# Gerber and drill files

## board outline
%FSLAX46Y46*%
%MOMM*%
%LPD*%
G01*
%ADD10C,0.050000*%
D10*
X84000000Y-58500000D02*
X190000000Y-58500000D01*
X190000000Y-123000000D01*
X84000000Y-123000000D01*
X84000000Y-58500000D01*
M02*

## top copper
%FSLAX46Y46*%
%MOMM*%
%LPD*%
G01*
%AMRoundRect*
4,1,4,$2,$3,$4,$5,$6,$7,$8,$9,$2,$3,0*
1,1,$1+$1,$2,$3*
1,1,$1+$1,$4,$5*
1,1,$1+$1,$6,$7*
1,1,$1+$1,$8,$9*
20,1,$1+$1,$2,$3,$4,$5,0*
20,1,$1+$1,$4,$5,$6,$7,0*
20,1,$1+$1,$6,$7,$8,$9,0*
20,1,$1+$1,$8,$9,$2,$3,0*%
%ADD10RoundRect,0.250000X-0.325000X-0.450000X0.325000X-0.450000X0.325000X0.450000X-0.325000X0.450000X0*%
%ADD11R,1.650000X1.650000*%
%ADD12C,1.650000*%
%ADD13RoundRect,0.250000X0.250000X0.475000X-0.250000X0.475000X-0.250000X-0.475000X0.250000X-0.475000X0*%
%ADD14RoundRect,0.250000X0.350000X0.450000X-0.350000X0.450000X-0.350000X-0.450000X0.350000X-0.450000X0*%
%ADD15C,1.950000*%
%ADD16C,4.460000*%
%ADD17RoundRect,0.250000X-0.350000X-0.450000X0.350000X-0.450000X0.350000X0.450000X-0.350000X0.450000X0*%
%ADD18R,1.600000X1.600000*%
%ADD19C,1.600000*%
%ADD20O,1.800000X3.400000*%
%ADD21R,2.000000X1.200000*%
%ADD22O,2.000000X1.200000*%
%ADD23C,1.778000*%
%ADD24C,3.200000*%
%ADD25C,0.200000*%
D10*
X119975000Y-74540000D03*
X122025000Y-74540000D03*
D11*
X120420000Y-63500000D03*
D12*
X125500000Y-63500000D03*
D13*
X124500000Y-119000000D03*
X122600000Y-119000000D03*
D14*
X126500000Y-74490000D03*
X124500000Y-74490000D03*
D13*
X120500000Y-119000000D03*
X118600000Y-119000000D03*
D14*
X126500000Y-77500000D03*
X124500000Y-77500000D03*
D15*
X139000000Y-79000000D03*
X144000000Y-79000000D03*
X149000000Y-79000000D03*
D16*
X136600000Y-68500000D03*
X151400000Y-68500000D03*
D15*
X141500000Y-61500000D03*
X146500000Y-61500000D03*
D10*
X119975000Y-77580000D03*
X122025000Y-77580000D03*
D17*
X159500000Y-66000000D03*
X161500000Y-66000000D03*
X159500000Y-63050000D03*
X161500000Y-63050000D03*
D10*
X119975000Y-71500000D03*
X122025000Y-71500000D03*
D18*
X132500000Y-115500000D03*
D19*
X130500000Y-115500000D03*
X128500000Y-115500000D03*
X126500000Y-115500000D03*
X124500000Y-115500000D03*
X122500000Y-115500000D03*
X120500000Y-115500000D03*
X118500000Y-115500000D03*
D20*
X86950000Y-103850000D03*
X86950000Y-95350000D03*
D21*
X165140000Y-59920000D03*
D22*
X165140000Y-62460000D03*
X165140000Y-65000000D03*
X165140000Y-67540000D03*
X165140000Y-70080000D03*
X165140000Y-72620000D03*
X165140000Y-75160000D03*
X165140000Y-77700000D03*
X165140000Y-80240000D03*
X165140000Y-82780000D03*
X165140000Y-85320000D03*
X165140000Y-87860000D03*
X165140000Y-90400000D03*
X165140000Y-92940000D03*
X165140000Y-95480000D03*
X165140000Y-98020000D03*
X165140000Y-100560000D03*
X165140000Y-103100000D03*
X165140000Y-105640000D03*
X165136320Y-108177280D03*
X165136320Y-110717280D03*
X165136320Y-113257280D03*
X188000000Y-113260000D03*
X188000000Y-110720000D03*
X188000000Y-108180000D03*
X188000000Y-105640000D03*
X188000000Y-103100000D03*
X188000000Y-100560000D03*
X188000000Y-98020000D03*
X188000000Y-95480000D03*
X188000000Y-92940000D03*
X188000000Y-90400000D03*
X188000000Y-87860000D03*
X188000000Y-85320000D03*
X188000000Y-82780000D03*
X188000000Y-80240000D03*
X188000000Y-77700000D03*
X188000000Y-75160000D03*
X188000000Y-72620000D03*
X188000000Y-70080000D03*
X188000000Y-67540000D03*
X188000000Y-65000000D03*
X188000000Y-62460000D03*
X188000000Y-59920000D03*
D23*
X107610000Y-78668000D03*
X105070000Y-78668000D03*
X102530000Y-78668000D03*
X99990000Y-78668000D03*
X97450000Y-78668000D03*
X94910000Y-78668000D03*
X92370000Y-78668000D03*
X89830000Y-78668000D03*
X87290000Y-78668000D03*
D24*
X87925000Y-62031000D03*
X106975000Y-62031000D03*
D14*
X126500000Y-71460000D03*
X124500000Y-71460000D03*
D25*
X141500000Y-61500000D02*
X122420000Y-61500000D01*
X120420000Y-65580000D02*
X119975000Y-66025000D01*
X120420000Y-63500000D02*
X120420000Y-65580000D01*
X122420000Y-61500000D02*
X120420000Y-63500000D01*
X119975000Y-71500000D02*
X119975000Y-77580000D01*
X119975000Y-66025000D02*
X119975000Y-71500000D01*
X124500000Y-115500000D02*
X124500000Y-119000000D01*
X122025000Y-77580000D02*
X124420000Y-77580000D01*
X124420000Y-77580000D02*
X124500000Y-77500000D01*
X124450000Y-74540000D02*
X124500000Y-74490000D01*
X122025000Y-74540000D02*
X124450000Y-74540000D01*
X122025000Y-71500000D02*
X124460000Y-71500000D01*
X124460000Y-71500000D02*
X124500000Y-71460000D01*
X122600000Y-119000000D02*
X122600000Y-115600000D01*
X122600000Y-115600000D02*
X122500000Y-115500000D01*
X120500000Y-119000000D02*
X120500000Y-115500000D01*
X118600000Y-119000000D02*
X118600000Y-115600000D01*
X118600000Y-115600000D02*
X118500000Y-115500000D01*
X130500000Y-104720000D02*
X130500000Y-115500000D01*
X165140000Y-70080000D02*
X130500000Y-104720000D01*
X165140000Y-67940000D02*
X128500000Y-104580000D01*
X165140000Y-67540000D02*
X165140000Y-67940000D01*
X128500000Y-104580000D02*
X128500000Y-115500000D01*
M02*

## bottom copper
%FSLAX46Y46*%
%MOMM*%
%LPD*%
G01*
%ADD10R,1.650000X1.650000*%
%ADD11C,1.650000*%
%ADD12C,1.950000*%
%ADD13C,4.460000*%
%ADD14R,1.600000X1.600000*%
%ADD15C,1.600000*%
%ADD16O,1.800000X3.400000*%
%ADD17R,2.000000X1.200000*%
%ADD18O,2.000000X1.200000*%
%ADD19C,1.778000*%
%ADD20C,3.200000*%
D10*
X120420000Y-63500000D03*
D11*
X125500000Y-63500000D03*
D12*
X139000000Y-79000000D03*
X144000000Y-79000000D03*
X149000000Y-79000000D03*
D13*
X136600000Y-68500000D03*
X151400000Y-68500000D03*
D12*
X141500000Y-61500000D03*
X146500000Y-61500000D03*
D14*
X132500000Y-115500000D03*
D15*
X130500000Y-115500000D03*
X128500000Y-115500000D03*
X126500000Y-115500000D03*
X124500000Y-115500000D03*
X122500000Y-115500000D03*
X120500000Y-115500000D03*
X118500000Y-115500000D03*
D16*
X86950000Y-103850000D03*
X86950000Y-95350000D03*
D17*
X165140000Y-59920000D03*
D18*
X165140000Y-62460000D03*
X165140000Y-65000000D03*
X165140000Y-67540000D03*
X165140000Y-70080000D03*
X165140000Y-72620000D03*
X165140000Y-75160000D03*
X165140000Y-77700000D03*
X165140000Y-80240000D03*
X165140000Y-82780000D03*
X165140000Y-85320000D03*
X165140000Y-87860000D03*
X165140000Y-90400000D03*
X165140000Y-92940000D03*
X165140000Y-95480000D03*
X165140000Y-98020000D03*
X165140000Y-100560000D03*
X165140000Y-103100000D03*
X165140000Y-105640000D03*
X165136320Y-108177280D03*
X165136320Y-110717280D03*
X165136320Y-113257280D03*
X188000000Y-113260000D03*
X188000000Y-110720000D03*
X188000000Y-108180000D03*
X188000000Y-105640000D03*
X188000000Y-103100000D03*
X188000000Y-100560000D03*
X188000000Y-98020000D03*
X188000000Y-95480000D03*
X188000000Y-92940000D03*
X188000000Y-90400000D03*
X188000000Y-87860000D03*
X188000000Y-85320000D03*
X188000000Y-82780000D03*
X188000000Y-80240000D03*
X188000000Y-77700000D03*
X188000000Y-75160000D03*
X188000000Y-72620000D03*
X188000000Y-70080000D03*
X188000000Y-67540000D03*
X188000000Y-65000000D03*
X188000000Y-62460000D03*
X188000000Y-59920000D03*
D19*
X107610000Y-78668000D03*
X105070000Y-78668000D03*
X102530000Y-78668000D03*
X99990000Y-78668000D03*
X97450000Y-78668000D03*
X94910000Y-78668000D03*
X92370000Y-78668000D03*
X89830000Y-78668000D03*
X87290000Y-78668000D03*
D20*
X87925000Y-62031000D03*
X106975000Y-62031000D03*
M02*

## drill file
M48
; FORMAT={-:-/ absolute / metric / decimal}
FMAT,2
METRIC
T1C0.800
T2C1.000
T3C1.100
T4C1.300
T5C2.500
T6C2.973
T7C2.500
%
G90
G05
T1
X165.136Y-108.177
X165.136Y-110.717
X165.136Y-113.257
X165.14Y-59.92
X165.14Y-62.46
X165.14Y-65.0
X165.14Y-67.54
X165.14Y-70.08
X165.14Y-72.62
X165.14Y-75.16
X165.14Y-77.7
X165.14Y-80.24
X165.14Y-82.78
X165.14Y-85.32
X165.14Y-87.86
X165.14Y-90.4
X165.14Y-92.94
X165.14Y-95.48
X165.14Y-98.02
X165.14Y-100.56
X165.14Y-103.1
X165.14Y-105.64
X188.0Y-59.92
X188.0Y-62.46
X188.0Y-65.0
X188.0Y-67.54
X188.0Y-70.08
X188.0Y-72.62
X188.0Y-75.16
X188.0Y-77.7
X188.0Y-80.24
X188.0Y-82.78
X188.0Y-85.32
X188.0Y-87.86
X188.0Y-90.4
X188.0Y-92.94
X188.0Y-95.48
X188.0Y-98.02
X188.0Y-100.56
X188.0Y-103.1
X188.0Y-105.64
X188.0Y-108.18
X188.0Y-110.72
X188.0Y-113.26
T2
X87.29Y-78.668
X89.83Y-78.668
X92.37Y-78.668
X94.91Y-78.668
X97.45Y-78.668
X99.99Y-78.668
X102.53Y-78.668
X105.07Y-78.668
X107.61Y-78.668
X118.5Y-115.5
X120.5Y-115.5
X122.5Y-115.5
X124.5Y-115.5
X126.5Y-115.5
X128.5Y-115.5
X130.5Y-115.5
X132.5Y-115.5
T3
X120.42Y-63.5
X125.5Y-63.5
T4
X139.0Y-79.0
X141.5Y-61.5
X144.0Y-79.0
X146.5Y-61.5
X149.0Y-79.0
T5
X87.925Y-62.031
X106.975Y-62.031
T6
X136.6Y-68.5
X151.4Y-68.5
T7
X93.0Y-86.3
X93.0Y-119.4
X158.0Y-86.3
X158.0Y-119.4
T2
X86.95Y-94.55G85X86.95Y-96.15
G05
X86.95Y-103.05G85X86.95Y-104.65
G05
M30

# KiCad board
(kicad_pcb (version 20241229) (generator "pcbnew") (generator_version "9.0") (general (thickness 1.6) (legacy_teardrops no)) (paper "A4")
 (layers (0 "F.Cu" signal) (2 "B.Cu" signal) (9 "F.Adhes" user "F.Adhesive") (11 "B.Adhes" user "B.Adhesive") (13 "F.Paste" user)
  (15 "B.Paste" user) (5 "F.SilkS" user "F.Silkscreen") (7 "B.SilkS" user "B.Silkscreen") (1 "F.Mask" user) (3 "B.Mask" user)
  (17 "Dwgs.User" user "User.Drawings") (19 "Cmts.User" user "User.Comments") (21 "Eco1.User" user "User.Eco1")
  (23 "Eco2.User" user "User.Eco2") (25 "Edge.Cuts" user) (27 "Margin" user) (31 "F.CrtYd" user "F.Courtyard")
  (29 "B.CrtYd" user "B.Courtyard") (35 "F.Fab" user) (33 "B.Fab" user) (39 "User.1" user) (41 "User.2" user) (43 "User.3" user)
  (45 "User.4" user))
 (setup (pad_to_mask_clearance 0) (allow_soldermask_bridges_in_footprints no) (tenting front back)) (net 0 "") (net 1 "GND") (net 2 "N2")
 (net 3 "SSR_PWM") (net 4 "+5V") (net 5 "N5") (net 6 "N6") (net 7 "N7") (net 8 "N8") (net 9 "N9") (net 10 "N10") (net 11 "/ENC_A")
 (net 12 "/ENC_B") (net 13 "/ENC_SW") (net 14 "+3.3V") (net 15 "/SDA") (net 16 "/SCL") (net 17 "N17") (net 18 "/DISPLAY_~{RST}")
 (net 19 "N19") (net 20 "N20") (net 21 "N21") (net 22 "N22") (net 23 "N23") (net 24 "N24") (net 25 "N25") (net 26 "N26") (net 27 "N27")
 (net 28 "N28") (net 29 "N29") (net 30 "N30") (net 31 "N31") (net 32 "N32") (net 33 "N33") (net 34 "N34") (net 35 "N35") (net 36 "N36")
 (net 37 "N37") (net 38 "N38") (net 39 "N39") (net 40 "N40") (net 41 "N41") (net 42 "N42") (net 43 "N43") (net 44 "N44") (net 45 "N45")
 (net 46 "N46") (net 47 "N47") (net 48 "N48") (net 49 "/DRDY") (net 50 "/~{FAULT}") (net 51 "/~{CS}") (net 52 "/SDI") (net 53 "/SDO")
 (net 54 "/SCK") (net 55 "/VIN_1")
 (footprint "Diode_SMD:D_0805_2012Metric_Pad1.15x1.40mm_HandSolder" (layer "F.Cu") (at 121 74.54)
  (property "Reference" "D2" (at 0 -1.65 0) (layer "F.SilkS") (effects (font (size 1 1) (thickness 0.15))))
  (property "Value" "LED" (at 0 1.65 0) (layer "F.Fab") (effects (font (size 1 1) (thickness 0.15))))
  (pad "1" smd roundrect (at -1.025 0) (size 1.15 1.4) (layers "F.Cu" "F.Mask" "F.Paste") (roundrect_rratio 0.217391) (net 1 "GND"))
  (pad "2" smd roundrect (at 1.025 0) (size 1.15 1.4) (layers "F.Cu" "F.Mask" "F.Paste") (roundrect_rratio 0.217391) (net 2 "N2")))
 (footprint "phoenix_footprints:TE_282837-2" (layer "F.Cu") (at 122.96 63.5)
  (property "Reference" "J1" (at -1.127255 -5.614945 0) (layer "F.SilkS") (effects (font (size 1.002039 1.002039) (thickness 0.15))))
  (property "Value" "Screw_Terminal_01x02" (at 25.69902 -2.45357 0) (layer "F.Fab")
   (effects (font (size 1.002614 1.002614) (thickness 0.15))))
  (pad "1" thru_hole rect (at -2.54 0) (size 1.65 1.65) (drill 1.1) (layers "*.Cu" "*.Mask") (remove_unused_layers no) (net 1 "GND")
   (solder_mask_margin 0.102))
  (pad "2" thru_hole circle (at 2.54 0) (size 1.65 1.65) (drill 1.1) (layers "*.Cu" "*.Mask") (remove_unused_layers no) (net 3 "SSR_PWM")
   (solder_mask_margin 0.102)))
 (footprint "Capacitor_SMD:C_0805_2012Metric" (layer "F.Cu") (at 123.55 119 180)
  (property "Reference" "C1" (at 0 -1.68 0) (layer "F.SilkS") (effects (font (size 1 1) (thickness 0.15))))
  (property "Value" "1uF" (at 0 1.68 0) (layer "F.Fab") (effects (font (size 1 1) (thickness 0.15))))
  (pad "1" smd roundrect (at -0.95 0 180) (size 1 1.45) (layers "F.Cu" "F.Mask" "F.Paste") (roundrect_rratio 0.25) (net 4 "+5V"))
  (pad "2" smd roundrect (at 0.95 0 180) (size 1 1.45) (layers "F.Cu" "F.Mask" "F.Paste") (roundrect_rratio 0.25) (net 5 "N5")))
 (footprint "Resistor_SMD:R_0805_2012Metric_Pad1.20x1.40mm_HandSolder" (layer "F.Cu") (at 125.5 74.49 180)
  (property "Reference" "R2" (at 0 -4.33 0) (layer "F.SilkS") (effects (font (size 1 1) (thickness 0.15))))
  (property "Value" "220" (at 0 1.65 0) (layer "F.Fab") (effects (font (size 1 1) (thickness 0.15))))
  (pad "1" smd roundrect (at -1 0 180) (size 1.2 1.4) (layers "F.Cu" "F.Mask" "F.Paste") (roundrect_rratio 0.208333) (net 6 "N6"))
  (pad "2" smd roundrect (at 1 0 180) (size 1.2 1.4) (layers "F.Cu" "F.Mask" "F.Paste") (roundrect_rratio 0.208333) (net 2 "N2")))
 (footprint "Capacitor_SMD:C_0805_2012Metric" (layer "F.Cu") (at 119.55 119 180)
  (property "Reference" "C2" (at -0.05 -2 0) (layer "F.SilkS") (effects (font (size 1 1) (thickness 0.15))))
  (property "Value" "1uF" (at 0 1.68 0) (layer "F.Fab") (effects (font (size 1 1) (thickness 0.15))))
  (pad "1" smd roundrect (at -0.95 0 180) (size 1 1.45) (layers "F.Cu" "F.Mask" "F.Paste") (roundrect_rratio 0.25) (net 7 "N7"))
  (pad "2" smd roundrect (at 0.95 0 180) (size 1 1.45) (layers "F.Cu" "F.Mask" "F.Paste") (roundrect_rratio 0.25) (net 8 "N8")))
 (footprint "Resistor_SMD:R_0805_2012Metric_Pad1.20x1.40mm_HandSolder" (layer "F.Cu") (at 125.5 77.5 180)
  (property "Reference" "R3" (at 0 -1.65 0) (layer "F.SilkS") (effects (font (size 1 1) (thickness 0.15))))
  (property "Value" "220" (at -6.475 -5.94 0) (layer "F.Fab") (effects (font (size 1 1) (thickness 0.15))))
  (pad "1" smd roundrect (at -1 0 180) (size 1.2 1.4) (layers "F.Cu" "F.Mask" "F.Paste") (roundrect_rratio 0.208333) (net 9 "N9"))
  (pad "2" smd roundrect (at 1 0 180) (size 1.2 1.4) (layers "F.Cu" "F.Mask" "F.Paste") (roundrect_rratio 0.208333) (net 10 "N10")))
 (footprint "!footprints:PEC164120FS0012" (layer "F.Cu") (at 139 79)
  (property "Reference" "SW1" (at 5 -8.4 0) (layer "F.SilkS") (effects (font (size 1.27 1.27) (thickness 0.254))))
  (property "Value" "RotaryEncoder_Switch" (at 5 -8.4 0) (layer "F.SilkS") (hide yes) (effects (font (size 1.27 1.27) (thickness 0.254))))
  (pad "A" thru_hole circle (at 0 0) (size 1.95 1.95) (drill 1.3) (layers "*.Cu" "*.Mask") (remove_unused_layers no) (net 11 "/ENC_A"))
  (pad "B" thru_hole circle (at 5 0) (size 1.95 1.95) (drill 1.3) (layers "*.Cu" "*.Mask") (remove_unused_layers no) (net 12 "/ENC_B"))
  (pad "C" thru_hole circle (at 10 0) (size 1.95 1.95) (drill 1.3) (layers "*.Cu" "*.Mask") (remove_unused_layers no) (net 1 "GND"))
  (pad "MH1" thru_hole circle (at -2.4 -10.5) (size 4.46 4.46) (drill 2.9732) (layers "*.Cu" "*.Mask") (remove_unused_layers no))
  (pad "MH2" thru_hole circle (at 12.4 -10.5) (size 4.46 4.46) (drill 2.9732) (layers "*.Cu" "*.Mask") (remove_unused_layers no))
  (pad "S1" thru_hole circle (at 2.5 -17.5) (size 1.95 1.95) (drill 1.3) (layers "*.Cu" "*.Mask") (remove_unused_layers no) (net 1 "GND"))
  (pad "S2" thru_hole circle (at 7.5 -17.5) (size 1.95 1.95) (drill 1.3) (layers "*.Cu" "*.Mask") (remove_unused_layers no)
   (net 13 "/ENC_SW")))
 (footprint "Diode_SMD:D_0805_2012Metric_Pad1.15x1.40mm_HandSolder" (layer "F.Cu") (at 121 77.58)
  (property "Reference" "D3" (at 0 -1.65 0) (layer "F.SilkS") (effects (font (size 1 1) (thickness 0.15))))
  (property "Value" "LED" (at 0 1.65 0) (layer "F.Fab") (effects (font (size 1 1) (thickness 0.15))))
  (pad "1" smd roundrect (at -1.025 0) (size 1.15 1.4) (layers "F.Cu" "F.Mask" "F.Paste") (roundrect_rratio 0.217391) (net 1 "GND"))
  (pad "2" smd roundrect (at 1.025 0) (size 1.15 1.4) (layers "F.Cu" "F.Mask" "F.Paste") (roundrect_rratio 0.217391) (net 10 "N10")))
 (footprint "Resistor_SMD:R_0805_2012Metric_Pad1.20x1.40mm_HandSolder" (layer "F.Cu") (at 160.5 66)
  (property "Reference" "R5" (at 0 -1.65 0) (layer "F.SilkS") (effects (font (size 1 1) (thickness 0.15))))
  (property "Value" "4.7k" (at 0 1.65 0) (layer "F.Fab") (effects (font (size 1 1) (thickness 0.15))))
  (pad "1" smd roundrect (at -1 0) (size 1.2 1.4) (layers "F.Cu" "F.Mask" "F.Paste") (roundrect_rratio 0.208333) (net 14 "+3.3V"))
  (pad "2" smd roundrect (at 1 0) (size 1.2 1.4) (layers "F.Cu" "F.Mask" "F.Paste") (roundrect_rratio 0.208333) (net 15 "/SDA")))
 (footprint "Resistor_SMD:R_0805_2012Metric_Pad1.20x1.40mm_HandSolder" (layer "F.Cu") (at 160.5 63.05)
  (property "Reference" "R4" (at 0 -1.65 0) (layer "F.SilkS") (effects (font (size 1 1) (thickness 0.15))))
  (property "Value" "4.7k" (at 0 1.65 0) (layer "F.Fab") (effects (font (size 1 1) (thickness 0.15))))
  (pad "1" smd roundrect (at -1 0) (size 1.2 1.4) (layers "F.Cu" "F.Mask" "F.Paste") (roundrect_rratio 0.208333) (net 14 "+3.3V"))
  (pad "2" smd roundrect (at 1 0) (size 1.2 1.4) (layers "F.Cu" "F.Mask" "F.Paste") (roundrect_rratio 0.208333) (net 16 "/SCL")))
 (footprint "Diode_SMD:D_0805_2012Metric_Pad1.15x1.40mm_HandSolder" (layer "F.Cu") (at 121 71.5)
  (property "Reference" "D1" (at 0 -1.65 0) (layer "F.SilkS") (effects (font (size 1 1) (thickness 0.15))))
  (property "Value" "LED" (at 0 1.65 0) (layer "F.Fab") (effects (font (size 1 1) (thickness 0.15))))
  (pad "1" smd roundrect (at -1.025 0) (size 1.15 1.4) (layers "F.Cu" "F.Mask" "F.Paste") (roundrect_rratio 0.217391) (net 1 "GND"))
  (pad "2" smd roundrect (at 1.025 0) (size 1.15 1.4) (layers "F.Cu" "F.Mask" "F.Paste") (roundrect_rratio 0.217391) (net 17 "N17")))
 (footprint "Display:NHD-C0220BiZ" (layer "F.Cu") (at 125.5 99.6)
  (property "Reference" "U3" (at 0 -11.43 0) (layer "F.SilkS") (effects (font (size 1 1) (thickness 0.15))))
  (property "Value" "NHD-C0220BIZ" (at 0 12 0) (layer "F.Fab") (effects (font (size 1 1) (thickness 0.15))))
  (pad "" np_thru_hole circle (at -32.5 -13.3) (size 2.5 2.5) (drill 2.5) (layers "*.Cu" "*.Mask"))
  (pad "" np_thru_hole circle (at -32.5 19.8) (size 2.5 2.5) (drill 2.5) (layers "*.Cu" "*.Mask"))
  (pad "" np_thru_hole circle (at 32.5 -13.3) (size 2.5 2.5) (drill 2.5) (layers "*.Cu" "*.Mask"))
  (pad "" np_thru_hole circle (at 32.5 19.8) (size 2.5 2.5) (drill 2.5) (layers "*.Cu" "*.Mask"))
  (pad "1" thru_hole rect (at 7 15.9) (size 1.6 1.6) (drill 1) (layers "*.Cu" "*.Mask") (remove_unused_layers no) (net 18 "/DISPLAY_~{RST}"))
  (pad "2" thru_hole circle (at 5 15.9) (size 1.6 1.6) (drill 1) (layers "*.Cu" "*.Mask") (remove_unused_layers no) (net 16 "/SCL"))
  (pad "3" thru_hole circle (at 3 15.9) (size 1.6 1.6) (drill 1) (layers "*.Cu" "*.Mask") (remove_unused_layers no) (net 15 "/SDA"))
  (pad "4" thru_hole circle (at 1 15.9) (size 1.6 1.6) (drill 1) (layers "*.Cu" "*.Mask") (remove_unused_layers no) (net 1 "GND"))
  (pad "5" thru_hole circle (at -1 15.9) (size 1.6 1.6) (drill 1) (layers "*.Cu" "*.Mask") (remove_unused_layers no) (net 4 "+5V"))
  (pad "6" thru_hole circle (at -3 15.9) (size 1.6 1.6) (drill 1) (layers "*.Cu" "*.Mask") (remove_unused_layers no) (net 5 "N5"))
  (pad "7" thru_hole circle (at -5 15.9) (size 1.6 1.6) (drill 1) (layers "*.Cu" "*.Mask") (remove_unused_layers no) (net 7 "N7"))
  (pad "8" thru_hole circle (at -7 15.9) (size 1.6 1.6) (drill 1) (layers "*.Cu" "*.Mask") (remove_unused_layers no) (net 8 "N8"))
  (pad "9" thru_hole oval (at -38.55 4.25) (size 1.8 3.4) (drill oval 1 2.6) (layers "*.Cu" "*.Mask") (remove_unused_layers no)
   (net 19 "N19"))
  (pad "10" thru_hole oval (at -38.55 -4.25) (size 1.8 3.4) (drill oval 1 2.6) (layers "*.Cu" "*.Mask") (remove_unused_layers no)
   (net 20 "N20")))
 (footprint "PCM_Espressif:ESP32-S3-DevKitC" (layer "F.Cu") (at 165.14 59.92)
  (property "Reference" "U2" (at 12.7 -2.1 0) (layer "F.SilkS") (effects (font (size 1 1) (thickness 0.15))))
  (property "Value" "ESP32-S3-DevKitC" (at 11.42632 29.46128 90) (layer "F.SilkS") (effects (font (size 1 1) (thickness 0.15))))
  (pad "1" thru_hole rect (at 0 0 270) (size 1.2 2) (drill 0.8) (layers "*.Cu" "*.Mask") (remove_unused_layers no) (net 14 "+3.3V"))
  (pad "2" thru_hole oval (at 0 2.54 270) (size 1.2 2) (drill 0.8) (layers "*.Cu" "*.Mask") (remove_unused_layers no) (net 14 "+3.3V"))
  (pad "3" thru_hole oval (at 0 5.08 270) (size 1.2 2) (drill 0.8) (layers "*.Cu" "*.Mask") (remove_unused_layers no) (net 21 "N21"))
  (pad "4" thru_hole oval (at 0 7.62 270) (size 1.2 2) (drill 0.8) (layers "*.Cu" "*.Mask") (remove_unused_layers no) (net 15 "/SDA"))
  (pad "5" thru_hole oval (at 0 10.16 270) (size 1.2 2) (drill 0.8) (layers "*.Cu" "*.Mask") (remove_unused_layers no) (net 16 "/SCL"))
  (pad "6" thru_hole oval (at 0 12.7 270) (size 1.2 2) (drill 0.8) (layers "*.Cu" "*.Mask") (remove_unused_layers no) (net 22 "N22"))
  (pad "7" thru_hole oval (at 0 15.24 270) (size 1.2 2) (drill 0.8) (layers "*.Cu" "*.Mask") (remove_unused_layers no) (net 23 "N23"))
  (pad "8" thru_hole oval (at 0 17.78 270) (size 1.2 2) (drill 0.8) (layers "*.Cu" "*.Mask") (remove_unused_layers no) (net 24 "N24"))
  (pad "9" thru_hole oval (at 0 20.32 270) (size 1.2 2) (drill 0.8) (layers "*.Cu" "*.Mask") (remove_unused_layers no) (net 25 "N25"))
  (pad "10" thru_hole oval (at 0 22.86 270) (size 1.2 2) (drill 0.8) (layers "*.Cu" "*.Mask") (remove_unused_layers no) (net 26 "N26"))
  (pad "11" thru_hole oval (at 0 25.4 270) (size 1.2 2) (drill 0.8) (layers "*.Cu" "*.Mask") (remove_unused_layers no) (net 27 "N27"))
  (pad "12" thru_hole oval (at 0 27.94 270) (size 1.2 2) (drill 0.8) (layers "*.Cu" "*.Mask") (remove_unused_layers no) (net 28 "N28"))
  (pad "13" thru_hole oval (at 0 30.48 270) (size 1.2 2) (drill 0.8) (layers "*.Cu" "*.Mask") (remove_unused_layers no) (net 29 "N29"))
  (pad "14" thru_hole oval (at 0 33.02 270) (size 1.2 2) (drill 0.8) (layers "*.Cu" "*.Mask") (remove_unused_layers no) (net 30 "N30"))
  (pad "15" thru_hole oval (at 0 35.56 270) (size 1.2 2) (drill 0.8) (layers "*.Cu" "*.Mask") (remove_unused_layers no) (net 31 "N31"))
  (pad "16" thru_hole oval (at 0 38.1 270) (size 1.2 2) (drill 0.8) (layers "*.Cu" "*.Mask") (remove_unused_layers no) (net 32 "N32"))
  (pad "17" thru_hole oval (at 0 40.64 270) (size 1.2 2) (drill 0.8) (layers "*.Cu" "*.Mask") (remove_unused_layers no) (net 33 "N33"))
  (pad "18" thru_hole oval (at 0 43.18 270) (size 1.2 2) (drill 0.8) (layers "*.Cu" "*.Mask") (remove_unused_layers no) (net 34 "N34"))
  (pad "19" thru_hole oval (at 0 45.72 270) (size 1.2 2) (drill 0.8) (layers "*.Cu" "*.Mask") (remove_unused_layers no) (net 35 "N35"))
  (pad "20" thru_hole oval (at -0.00368 48.25728 270) (size 1.2 2) (drill 0.8) (layers "*.Cu" "*.Mask") (remove_unused_layers no)
   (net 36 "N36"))
  (pad "21" thru_hole oval (at -0.00368 50.79728 270) (size 1.2 2) (drill 0.8) (layers "*.Cu" "*.Mask") (remove_unused_layers no)
   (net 4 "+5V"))
  (pad "22" thru_hole oval (at -0.00368 53.33728 270) (size 1.2 2) (drill 0.8) (layers "*.Cu" "*.Mask") (remove_unused_layers no)
   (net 1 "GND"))
  (pad "23" thru_hole oval (at 22.86 53.34 270) (size 1.2 2) (drill 0.8) (layers "*.Cu" "*.Mask") (remove_unused_layers no) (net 1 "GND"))
  (pad "24" thru_hole oval (at 22.86 50.8 270) (size 1.2 2) (drill 0.8) (layers "*.Cu" "*.Mask") (remove_unused_layers no) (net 1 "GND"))
  (pad "25" thru_hole oval (at 22.86 48.26 270) (size 1.2 2) (drill 0.8) (layers "*.Cu" "*.Mask") (remove_unused_layers no) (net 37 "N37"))
  (pad "26" thru_hole oval (at 22.86 45.72 270) (size 1.2 2) (drill 0.8) (layers "*.Cu" "*.Mask") (remove_unused_layers no) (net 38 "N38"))
  (pad "27" thru_hole oval (at 22.86 43.18 270) (size 1.2 2) (drill 0.8) (layers "*.Cu" "*.Mask") (remove_unused_layers no)
   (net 3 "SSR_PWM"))
  (pad "28" thru_hole oval (at 22.86 40.64 270) (size 1.2 2) (drill 0.8) (layers "*.Cu" "*.Mask") (remove_unused_layers no) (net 6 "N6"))
  (pad "29" thru_hole oval (at 22.86 38.1 270) (size 1.2 2) (drill 0.8) (layers "*.Cu" "*.Mask") (remove_unused_layers no) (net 9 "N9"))
  (pad "30" thru_hole oval (at 22.86 35.56 270) (size 1.2 2) (drill 0.8) (layers "*.Cu" "*.Mask") (remove_unused_layers no) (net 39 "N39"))
  (pad "31" thru_hole oval (at 22.86 33.02 270) (size 1.2 2) (drill 0.8) (layers "*.Cu" "*.Mask") (remove_unused_layers no) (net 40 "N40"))
  (pad "32" thru_hole oval (at 22.86 30.48 270) (size 1.2 2) (drill 0.8) (layers "*.Cu" "*.Mask") (remove_unused_layers no)
   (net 18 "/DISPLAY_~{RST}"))
  (pad "33" thru_hole oval (at 22.86 27.94 270) (size 1.2 2) (drill 0.8) (layers "*.Cu" "*.Mask") (remove_unused_layers no)
   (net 11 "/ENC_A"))
  (pad "34" thru_hole oval (at 22.86 25.4 270) (size 1.2 2) (drill 0.8) (layers "*.Cu" "*.Mask") (remove_unused_layers no) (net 12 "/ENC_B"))
  (pad "35" thru_hole oval (at 22.86 22.86 270) (size 1.2 2) (drill 0.8) (layers "*.Cu" "*.Mask") (remove_unused_layers no)
   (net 13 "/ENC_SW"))
  (pad "36" thru_hole oval (at 22.86 20.32 270) (size 1.2 2) (drill 0.8) (layers "*.Cu" "*.Mask") (remove_unused_layers no) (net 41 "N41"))
  (pad "37" thru_hole oval (at 22.86 17.78 270) (size 1.2 2) (drill 0.8) (layers "*.Cu" "*.Mask") (remove_unused_layers no) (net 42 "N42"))
  (pad "38" thru_hole oval (at 22.86 15.24 270) (size 1.2 2) (drill 0.8) (layers "*.Cu" "*.Mask") (remove_unused_layers no) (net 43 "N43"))
  (pad "39" thru_hole oval (at 22.86 12.7 270) (size 1.2 2) (drill 0.8) (layers "*.Cu" "*.Mask") (remove_unused_layers no) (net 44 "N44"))
  (pad "40" thru_hole oval (at 22.86 10.16 270) (size 1.2 2) (drill 0.8) (layers "*.Cu" "*.Mask") (remove_unused_layers no) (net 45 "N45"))
  (pad "41" thru_hole oval (at 22.86 7.62 270) (size 1.2 2) (drill 0.8) (layers "*.Cu" "*.Mask") (remove_unused_layers no) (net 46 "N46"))
  (pad "42" thru_hole oval (at 22.86 5.08 270) (size 1.2 2) (drill 0.8) (layers "*.Cu" "*.Mask") (remove_unused_layers no) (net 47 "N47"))
  (pad "43" thru_hole oval (at 22.86 2.54 270) (size 1.2 2) (drill 0.8) (layers "*.Cu" "*.Mask") (remove_unused_layers no) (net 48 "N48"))
  (pad "44" thru_hole oval (at 22.86 0 270) (size 1.2 2) (drill 0.8) (layers "*.Cu" "*.Mask") (remove_unused_layers no) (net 1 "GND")))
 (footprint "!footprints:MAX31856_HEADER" (layer "F.Cu") (at 87.936314 62.019686)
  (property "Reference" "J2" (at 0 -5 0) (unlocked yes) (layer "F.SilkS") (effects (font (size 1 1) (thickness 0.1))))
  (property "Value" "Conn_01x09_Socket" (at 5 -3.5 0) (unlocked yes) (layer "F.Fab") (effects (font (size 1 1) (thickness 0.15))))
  (pad "1" thru_hole circle (at 19.673686 16.648314 270) (size 1.778 1.778) (drill 1) (layers "*.Cu" "*.Mask") (remove_unused_layers no)
   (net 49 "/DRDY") (solder_mask_margin 0.0508) (thermal_bridge_angle 0))
  (pad "2" thru_hole circle (at 17.133686 16.648314 270) (size 1.778 1.778) (drill 1) (layers "*.Cu" "*.Mask") (remove_unused_layers no)
   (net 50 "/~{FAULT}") (solder_mask_margin 0.0508) (thermal_bridge_angle 0))
  (pad "3" thru_hole circle (at 14.593686 16.648314 270) (size 1.778 1.778) (drill 1) (layers "*.Cu" "*.Mask") (remove_unused_layers no)
   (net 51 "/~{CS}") (solder_mask_margin 0.0508) (thermal_bridge_angle 0))
  (pad "4" thru_hole circle (at 12.053686 16.648314 270) (size 1.778 1.778) (drill 1) (layers "*.Cu" "*.Mask") (remove_unused_layers no)
   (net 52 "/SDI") (solder_mask_margin 0.0508) (thermal_bridge_angle 0))
  (pad "5" thru_hole circle (at 9.513686 16.648314 270) (size 1.778 1.778) (drill 1) (layers "*.Cu" "*.Mask") (remove_unused_layers no)
   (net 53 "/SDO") (solder_mask_margin 0.0508) (thermal_bridge_angle 0))
  (pad "6" thru_hole circle (at 6.973686 16.648314 270) (size 1.778 1.778) (drill 1) (layers "*.Cu" "*.Mask") (remove_unused_layers no)
   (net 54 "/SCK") (solder_mask_margin 0.0508) (thermal_bridge_angle 0))
  (pad "7" thru_hole circle (at 4.433686 16.648314 270) (size 1.778 1.778) (drill 1) (layers "*.Cu" "*.Mask") (remove_unused_layers no)
   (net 1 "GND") (solder_mask_margin 0.0508) (thermal_bridge_angle 0))
  (pad "8" thru_hole circle (at 1.893686 16.648314 270) (size 1.778 1.778) (drill 1) (layers "*.Cu" "*.Mask") (remove_unused_layers no)
   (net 14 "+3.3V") (solder_mask_margin 0.0508) (thermal_bridge_angle 0))
  (pad "9" thru_hole circle (at -0.646314 16.648314 270) (size 1.778 1.778) (drill 1) (layers "*.Cu" "*.Mask") (remove_unused_layers no)
   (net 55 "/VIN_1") (solder_mask_margin 0.0508) (thermal_bridge_angle 0))
  (pad "P$1" thru_hole circle (at -0.011314 0.011314) (size 3.2 3.2) (drill 2.5) (layers "*.Cu" "*.Mask") (remove_unused_layers no)
   (solder_mask_margin 0.0508) (thermal_bridge_angle 0))
  (pad "P$1" thru_hole circle (at 19.038686 0.011314) (size 3.2 3.2) (drill 2.5) (layers "*.Cu" "*.Mask") (remove_unused_layers no)
   (solder_mask_margin 0.0508) (thermal_bridge_angle 0))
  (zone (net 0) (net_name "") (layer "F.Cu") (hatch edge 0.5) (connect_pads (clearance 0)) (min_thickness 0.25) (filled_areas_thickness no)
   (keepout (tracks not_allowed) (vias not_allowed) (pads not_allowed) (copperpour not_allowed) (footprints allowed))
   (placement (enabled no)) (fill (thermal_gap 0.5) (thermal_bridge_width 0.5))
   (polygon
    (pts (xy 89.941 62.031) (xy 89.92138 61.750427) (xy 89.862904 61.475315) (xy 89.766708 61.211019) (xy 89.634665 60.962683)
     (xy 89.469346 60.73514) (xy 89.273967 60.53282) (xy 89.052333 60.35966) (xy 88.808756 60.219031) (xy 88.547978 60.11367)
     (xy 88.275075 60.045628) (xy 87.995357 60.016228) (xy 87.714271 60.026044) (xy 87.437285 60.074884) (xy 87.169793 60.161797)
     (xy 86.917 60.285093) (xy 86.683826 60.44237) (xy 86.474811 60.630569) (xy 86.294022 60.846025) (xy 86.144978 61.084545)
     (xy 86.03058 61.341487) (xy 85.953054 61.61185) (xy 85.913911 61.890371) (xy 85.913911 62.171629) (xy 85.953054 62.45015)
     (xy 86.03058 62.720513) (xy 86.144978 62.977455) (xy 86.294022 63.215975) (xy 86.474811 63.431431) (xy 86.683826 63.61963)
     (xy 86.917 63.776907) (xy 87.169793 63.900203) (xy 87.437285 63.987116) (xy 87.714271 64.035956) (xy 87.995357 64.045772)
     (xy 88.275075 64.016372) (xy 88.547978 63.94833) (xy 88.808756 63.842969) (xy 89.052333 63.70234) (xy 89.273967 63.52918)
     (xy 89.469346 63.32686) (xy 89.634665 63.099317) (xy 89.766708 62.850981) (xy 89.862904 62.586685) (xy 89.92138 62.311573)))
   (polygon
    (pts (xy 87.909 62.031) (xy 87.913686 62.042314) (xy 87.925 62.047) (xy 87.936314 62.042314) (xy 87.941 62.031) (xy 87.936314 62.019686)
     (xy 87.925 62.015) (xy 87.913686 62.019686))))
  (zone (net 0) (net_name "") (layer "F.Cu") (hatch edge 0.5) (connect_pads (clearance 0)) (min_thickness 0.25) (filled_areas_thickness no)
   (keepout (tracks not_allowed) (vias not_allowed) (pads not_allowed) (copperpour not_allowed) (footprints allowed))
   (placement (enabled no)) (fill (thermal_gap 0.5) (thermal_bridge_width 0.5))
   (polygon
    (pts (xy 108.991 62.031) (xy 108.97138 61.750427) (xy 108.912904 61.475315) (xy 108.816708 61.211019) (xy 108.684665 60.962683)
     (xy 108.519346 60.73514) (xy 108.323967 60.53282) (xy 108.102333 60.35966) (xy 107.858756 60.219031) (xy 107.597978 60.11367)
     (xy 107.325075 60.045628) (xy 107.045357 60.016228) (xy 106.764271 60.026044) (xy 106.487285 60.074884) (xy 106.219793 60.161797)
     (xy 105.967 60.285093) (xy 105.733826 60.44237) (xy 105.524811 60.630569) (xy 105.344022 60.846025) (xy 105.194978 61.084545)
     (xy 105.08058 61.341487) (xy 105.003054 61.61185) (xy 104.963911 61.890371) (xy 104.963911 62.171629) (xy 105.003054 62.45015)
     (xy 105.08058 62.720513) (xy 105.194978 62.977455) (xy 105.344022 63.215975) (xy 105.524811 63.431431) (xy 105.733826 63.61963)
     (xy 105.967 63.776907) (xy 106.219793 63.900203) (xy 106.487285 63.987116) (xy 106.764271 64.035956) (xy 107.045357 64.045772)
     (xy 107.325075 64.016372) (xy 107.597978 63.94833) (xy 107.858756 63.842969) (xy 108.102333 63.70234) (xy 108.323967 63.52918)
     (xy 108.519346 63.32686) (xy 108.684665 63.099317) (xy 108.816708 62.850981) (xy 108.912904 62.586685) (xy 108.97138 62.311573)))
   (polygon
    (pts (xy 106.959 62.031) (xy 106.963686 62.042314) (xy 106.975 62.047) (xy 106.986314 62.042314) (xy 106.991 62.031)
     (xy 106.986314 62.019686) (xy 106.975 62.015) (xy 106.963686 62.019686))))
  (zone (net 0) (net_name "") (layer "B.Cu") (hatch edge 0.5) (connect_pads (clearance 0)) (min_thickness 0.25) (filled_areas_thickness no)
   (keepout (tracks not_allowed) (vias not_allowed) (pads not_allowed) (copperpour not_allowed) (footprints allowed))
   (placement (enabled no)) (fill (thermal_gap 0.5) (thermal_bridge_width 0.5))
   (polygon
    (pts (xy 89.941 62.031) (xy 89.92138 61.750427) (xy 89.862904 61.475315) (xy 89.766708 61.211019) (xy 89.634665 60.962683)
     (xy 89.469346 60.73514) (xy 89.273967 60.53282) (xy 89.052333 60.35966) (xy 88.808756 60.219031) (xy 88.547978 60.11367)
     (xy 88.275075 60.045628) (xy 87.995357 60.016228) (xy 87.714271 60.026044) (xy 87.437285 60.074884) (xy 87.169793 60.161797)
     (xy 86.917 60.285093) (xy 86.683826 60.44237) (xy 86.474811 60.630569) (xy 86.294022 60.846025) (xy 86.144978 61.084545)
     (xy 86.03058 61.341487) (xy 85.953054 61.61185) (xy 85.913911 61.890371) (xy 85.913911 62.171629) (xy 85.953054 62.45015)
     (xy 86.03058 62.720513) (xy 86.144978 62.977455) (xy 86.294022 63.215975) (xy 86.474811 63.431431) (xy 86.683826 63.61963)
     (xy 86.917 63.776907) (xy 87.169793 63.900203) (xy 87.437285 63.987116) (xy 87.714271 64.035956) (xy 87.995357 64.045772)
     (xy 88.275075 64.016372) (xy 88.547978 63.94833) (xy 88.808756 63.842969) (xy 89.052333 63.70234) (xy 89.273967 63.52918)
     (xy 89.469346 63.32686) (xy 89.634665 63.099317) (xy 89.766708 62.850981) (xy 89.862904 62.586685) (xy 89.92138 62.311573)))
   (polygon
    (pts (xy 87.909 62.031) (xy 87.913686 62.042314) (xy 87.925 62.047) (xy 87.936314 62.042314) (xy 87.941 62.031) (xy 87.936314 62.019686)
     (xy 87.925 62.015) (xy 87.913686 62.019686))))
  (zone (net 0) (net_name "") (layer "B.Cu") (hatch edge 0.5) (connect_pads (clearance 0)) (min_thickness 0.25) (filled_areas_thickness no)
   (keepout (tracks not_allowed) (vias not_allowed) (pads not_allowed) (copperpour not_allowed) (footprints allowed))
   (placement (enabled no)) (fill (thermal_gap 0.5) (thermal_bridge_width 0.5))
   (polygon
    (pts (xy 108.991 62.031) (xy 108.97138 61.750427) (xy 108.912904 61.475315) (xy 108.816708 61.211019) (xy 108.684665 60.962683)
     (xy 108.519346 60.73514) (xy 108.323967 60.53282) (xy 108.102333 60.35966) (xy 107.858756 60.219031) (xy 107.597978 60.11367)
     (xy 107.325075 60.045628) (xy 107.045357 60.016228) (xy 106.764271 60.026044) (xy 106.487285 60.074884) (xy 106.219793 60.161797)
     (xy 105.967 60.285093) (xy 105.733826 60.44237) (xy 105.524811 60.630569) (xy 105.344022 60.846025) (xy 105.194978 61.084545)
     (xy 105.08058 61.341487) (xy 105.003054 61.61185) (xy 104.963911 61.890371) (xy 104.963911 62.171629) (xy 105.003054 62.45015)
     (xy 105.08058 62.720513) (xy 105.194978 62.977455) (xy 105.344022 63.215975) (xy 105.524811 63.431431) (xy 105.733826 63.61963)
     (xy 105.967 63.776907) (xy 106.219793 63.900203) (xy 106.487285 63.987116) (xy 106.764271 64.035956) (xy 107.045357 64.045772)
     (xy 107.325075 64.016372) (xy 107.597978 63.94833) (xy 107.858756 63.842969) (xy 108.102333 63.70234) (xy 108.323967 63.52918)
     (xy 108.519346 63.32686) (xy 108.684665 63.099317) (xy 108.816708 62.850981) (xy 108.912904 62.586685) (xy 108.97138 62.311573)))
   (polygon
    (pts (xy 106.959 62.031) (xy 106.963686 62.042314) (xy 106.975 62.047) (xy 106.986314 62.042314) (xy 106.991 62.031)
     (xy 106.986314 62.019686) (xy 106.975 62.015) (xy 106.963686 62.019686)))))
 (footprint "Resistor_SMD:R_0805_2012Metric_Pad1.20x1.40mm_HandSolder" (layer "F.Cu") (at 125.5 71.46 180)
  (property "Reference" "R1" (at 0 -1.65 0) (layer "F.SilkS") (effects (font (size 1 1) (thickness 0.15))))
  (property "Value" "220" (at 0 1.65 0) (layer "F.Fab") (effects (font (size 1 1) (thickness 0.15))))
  (pad "1" smd roundrect (at -1 0 180) (size 1.2 1.4) (layers "F.Cu" "F.Mask" "F.Paste") (roundrect_rratio 0.208333) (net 30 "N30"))
  (pad "2" smd roundrect (at 1 0 180) (size 1.2 1.4) (layers "F.Cu" "F.Mask" "F.Paste") (roundrect_rratio 0.208333) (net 17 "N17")))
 (gr_rect (start 84 58.5) (end 190 123) (stroke (width 0.05) (type default)) (fill no) (layer "Edge.Cuts"))
 (segment (start 141.5 61.5) (end 122.42 61.5) (width 0.2) (layer "F.Cu") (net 1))
 (segment (start 120.42 65.58) (end 119.975 66.025) (width 0.2) (layer "F.Cu") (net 1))
 (segment (start 120.42 63.5) (end 120.42 65.58) (width 0.2) (layer "F.Cu") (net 1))
 (segment (start 122.42 61.5) (end 120.42 63.5) (width 0.2) (layer "F.Cu") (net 1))
 (segment (start 119.975 71.5) (end 119.975 77.58) (width 0.2) (layer "F.Cu") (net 1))
 (segment (start 119.975 66.025) (end 119.975 71.5) (width 0.2) (layer "F.Cu") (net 1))
 (segment (start 124.5 115.5) (end 124.5 119) (width 0.2) (layer "F.Cu") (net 4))
 (segment (start 122.025 77.58) (end 124.42 77.58) (width 0.2) (layer "F.Cu") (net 10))
 (segment (start 124.42 77.58) (end 124.5 77.5) (width 0.2) (layer "F.Cu") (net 10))
 (segment (start 124.45 74.54) (end 124.5 74.49) (width 0.2) (layer "F.Cu") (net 2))
 (segment (start 122.025 74.54) (end 124.45 74.54) (width 0.2) (layer "F.Cu") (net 2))
 (segment (start 122.025 71.5) (end 124.46 71.5) (width 0.2) (layer "F.Cu") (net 17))
 (segment (start 124.46 71.5) (end 124.5 71.46) (width 0.2) (layer "F.Cu") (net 17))
 (segment (start 122.6 119) (end 122.6 115.6) (width 0.2) (layer "F.Cu") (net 5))
 (segment (start 122.6 115.6) (end 122.5 115.5) (width 0.2) (layer "F.Cu") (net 5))
 (segment (start 120.5 119) (end 120.5 115.5) (width 0.2) (layer "F.Cu") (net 7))
 (segment (start 118.6 119) (end 118.6 115.6) (width 0.2) (layer "F.Cu") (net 8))
 (segment (start 118.6 115.6) (end 118.5 115.5) (width 0.2) (layer "F.Cu") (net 8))
 (segment (start 130.5 104.72) (end 130.5 115.5) (width 0.2) (layer "F.Cu") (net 16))
 (segment (start 165.14 70.08) (end 130.5 104.72) (width 0.2) (layer "F.Cu") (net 16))
 (segment (start 165.14 67.94) (end 128.5 104.58) (width 0.2) (layer "F.Cu") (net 15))
 (segment (start 165.14 67.54) (end 165.14 67.94) (width 0.2) (layer "F.Cu") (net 15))
 (segment (start 128.5 104.58) (end 128.5 115.5) (width 0.2) (layer "F.Cu") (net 15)))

